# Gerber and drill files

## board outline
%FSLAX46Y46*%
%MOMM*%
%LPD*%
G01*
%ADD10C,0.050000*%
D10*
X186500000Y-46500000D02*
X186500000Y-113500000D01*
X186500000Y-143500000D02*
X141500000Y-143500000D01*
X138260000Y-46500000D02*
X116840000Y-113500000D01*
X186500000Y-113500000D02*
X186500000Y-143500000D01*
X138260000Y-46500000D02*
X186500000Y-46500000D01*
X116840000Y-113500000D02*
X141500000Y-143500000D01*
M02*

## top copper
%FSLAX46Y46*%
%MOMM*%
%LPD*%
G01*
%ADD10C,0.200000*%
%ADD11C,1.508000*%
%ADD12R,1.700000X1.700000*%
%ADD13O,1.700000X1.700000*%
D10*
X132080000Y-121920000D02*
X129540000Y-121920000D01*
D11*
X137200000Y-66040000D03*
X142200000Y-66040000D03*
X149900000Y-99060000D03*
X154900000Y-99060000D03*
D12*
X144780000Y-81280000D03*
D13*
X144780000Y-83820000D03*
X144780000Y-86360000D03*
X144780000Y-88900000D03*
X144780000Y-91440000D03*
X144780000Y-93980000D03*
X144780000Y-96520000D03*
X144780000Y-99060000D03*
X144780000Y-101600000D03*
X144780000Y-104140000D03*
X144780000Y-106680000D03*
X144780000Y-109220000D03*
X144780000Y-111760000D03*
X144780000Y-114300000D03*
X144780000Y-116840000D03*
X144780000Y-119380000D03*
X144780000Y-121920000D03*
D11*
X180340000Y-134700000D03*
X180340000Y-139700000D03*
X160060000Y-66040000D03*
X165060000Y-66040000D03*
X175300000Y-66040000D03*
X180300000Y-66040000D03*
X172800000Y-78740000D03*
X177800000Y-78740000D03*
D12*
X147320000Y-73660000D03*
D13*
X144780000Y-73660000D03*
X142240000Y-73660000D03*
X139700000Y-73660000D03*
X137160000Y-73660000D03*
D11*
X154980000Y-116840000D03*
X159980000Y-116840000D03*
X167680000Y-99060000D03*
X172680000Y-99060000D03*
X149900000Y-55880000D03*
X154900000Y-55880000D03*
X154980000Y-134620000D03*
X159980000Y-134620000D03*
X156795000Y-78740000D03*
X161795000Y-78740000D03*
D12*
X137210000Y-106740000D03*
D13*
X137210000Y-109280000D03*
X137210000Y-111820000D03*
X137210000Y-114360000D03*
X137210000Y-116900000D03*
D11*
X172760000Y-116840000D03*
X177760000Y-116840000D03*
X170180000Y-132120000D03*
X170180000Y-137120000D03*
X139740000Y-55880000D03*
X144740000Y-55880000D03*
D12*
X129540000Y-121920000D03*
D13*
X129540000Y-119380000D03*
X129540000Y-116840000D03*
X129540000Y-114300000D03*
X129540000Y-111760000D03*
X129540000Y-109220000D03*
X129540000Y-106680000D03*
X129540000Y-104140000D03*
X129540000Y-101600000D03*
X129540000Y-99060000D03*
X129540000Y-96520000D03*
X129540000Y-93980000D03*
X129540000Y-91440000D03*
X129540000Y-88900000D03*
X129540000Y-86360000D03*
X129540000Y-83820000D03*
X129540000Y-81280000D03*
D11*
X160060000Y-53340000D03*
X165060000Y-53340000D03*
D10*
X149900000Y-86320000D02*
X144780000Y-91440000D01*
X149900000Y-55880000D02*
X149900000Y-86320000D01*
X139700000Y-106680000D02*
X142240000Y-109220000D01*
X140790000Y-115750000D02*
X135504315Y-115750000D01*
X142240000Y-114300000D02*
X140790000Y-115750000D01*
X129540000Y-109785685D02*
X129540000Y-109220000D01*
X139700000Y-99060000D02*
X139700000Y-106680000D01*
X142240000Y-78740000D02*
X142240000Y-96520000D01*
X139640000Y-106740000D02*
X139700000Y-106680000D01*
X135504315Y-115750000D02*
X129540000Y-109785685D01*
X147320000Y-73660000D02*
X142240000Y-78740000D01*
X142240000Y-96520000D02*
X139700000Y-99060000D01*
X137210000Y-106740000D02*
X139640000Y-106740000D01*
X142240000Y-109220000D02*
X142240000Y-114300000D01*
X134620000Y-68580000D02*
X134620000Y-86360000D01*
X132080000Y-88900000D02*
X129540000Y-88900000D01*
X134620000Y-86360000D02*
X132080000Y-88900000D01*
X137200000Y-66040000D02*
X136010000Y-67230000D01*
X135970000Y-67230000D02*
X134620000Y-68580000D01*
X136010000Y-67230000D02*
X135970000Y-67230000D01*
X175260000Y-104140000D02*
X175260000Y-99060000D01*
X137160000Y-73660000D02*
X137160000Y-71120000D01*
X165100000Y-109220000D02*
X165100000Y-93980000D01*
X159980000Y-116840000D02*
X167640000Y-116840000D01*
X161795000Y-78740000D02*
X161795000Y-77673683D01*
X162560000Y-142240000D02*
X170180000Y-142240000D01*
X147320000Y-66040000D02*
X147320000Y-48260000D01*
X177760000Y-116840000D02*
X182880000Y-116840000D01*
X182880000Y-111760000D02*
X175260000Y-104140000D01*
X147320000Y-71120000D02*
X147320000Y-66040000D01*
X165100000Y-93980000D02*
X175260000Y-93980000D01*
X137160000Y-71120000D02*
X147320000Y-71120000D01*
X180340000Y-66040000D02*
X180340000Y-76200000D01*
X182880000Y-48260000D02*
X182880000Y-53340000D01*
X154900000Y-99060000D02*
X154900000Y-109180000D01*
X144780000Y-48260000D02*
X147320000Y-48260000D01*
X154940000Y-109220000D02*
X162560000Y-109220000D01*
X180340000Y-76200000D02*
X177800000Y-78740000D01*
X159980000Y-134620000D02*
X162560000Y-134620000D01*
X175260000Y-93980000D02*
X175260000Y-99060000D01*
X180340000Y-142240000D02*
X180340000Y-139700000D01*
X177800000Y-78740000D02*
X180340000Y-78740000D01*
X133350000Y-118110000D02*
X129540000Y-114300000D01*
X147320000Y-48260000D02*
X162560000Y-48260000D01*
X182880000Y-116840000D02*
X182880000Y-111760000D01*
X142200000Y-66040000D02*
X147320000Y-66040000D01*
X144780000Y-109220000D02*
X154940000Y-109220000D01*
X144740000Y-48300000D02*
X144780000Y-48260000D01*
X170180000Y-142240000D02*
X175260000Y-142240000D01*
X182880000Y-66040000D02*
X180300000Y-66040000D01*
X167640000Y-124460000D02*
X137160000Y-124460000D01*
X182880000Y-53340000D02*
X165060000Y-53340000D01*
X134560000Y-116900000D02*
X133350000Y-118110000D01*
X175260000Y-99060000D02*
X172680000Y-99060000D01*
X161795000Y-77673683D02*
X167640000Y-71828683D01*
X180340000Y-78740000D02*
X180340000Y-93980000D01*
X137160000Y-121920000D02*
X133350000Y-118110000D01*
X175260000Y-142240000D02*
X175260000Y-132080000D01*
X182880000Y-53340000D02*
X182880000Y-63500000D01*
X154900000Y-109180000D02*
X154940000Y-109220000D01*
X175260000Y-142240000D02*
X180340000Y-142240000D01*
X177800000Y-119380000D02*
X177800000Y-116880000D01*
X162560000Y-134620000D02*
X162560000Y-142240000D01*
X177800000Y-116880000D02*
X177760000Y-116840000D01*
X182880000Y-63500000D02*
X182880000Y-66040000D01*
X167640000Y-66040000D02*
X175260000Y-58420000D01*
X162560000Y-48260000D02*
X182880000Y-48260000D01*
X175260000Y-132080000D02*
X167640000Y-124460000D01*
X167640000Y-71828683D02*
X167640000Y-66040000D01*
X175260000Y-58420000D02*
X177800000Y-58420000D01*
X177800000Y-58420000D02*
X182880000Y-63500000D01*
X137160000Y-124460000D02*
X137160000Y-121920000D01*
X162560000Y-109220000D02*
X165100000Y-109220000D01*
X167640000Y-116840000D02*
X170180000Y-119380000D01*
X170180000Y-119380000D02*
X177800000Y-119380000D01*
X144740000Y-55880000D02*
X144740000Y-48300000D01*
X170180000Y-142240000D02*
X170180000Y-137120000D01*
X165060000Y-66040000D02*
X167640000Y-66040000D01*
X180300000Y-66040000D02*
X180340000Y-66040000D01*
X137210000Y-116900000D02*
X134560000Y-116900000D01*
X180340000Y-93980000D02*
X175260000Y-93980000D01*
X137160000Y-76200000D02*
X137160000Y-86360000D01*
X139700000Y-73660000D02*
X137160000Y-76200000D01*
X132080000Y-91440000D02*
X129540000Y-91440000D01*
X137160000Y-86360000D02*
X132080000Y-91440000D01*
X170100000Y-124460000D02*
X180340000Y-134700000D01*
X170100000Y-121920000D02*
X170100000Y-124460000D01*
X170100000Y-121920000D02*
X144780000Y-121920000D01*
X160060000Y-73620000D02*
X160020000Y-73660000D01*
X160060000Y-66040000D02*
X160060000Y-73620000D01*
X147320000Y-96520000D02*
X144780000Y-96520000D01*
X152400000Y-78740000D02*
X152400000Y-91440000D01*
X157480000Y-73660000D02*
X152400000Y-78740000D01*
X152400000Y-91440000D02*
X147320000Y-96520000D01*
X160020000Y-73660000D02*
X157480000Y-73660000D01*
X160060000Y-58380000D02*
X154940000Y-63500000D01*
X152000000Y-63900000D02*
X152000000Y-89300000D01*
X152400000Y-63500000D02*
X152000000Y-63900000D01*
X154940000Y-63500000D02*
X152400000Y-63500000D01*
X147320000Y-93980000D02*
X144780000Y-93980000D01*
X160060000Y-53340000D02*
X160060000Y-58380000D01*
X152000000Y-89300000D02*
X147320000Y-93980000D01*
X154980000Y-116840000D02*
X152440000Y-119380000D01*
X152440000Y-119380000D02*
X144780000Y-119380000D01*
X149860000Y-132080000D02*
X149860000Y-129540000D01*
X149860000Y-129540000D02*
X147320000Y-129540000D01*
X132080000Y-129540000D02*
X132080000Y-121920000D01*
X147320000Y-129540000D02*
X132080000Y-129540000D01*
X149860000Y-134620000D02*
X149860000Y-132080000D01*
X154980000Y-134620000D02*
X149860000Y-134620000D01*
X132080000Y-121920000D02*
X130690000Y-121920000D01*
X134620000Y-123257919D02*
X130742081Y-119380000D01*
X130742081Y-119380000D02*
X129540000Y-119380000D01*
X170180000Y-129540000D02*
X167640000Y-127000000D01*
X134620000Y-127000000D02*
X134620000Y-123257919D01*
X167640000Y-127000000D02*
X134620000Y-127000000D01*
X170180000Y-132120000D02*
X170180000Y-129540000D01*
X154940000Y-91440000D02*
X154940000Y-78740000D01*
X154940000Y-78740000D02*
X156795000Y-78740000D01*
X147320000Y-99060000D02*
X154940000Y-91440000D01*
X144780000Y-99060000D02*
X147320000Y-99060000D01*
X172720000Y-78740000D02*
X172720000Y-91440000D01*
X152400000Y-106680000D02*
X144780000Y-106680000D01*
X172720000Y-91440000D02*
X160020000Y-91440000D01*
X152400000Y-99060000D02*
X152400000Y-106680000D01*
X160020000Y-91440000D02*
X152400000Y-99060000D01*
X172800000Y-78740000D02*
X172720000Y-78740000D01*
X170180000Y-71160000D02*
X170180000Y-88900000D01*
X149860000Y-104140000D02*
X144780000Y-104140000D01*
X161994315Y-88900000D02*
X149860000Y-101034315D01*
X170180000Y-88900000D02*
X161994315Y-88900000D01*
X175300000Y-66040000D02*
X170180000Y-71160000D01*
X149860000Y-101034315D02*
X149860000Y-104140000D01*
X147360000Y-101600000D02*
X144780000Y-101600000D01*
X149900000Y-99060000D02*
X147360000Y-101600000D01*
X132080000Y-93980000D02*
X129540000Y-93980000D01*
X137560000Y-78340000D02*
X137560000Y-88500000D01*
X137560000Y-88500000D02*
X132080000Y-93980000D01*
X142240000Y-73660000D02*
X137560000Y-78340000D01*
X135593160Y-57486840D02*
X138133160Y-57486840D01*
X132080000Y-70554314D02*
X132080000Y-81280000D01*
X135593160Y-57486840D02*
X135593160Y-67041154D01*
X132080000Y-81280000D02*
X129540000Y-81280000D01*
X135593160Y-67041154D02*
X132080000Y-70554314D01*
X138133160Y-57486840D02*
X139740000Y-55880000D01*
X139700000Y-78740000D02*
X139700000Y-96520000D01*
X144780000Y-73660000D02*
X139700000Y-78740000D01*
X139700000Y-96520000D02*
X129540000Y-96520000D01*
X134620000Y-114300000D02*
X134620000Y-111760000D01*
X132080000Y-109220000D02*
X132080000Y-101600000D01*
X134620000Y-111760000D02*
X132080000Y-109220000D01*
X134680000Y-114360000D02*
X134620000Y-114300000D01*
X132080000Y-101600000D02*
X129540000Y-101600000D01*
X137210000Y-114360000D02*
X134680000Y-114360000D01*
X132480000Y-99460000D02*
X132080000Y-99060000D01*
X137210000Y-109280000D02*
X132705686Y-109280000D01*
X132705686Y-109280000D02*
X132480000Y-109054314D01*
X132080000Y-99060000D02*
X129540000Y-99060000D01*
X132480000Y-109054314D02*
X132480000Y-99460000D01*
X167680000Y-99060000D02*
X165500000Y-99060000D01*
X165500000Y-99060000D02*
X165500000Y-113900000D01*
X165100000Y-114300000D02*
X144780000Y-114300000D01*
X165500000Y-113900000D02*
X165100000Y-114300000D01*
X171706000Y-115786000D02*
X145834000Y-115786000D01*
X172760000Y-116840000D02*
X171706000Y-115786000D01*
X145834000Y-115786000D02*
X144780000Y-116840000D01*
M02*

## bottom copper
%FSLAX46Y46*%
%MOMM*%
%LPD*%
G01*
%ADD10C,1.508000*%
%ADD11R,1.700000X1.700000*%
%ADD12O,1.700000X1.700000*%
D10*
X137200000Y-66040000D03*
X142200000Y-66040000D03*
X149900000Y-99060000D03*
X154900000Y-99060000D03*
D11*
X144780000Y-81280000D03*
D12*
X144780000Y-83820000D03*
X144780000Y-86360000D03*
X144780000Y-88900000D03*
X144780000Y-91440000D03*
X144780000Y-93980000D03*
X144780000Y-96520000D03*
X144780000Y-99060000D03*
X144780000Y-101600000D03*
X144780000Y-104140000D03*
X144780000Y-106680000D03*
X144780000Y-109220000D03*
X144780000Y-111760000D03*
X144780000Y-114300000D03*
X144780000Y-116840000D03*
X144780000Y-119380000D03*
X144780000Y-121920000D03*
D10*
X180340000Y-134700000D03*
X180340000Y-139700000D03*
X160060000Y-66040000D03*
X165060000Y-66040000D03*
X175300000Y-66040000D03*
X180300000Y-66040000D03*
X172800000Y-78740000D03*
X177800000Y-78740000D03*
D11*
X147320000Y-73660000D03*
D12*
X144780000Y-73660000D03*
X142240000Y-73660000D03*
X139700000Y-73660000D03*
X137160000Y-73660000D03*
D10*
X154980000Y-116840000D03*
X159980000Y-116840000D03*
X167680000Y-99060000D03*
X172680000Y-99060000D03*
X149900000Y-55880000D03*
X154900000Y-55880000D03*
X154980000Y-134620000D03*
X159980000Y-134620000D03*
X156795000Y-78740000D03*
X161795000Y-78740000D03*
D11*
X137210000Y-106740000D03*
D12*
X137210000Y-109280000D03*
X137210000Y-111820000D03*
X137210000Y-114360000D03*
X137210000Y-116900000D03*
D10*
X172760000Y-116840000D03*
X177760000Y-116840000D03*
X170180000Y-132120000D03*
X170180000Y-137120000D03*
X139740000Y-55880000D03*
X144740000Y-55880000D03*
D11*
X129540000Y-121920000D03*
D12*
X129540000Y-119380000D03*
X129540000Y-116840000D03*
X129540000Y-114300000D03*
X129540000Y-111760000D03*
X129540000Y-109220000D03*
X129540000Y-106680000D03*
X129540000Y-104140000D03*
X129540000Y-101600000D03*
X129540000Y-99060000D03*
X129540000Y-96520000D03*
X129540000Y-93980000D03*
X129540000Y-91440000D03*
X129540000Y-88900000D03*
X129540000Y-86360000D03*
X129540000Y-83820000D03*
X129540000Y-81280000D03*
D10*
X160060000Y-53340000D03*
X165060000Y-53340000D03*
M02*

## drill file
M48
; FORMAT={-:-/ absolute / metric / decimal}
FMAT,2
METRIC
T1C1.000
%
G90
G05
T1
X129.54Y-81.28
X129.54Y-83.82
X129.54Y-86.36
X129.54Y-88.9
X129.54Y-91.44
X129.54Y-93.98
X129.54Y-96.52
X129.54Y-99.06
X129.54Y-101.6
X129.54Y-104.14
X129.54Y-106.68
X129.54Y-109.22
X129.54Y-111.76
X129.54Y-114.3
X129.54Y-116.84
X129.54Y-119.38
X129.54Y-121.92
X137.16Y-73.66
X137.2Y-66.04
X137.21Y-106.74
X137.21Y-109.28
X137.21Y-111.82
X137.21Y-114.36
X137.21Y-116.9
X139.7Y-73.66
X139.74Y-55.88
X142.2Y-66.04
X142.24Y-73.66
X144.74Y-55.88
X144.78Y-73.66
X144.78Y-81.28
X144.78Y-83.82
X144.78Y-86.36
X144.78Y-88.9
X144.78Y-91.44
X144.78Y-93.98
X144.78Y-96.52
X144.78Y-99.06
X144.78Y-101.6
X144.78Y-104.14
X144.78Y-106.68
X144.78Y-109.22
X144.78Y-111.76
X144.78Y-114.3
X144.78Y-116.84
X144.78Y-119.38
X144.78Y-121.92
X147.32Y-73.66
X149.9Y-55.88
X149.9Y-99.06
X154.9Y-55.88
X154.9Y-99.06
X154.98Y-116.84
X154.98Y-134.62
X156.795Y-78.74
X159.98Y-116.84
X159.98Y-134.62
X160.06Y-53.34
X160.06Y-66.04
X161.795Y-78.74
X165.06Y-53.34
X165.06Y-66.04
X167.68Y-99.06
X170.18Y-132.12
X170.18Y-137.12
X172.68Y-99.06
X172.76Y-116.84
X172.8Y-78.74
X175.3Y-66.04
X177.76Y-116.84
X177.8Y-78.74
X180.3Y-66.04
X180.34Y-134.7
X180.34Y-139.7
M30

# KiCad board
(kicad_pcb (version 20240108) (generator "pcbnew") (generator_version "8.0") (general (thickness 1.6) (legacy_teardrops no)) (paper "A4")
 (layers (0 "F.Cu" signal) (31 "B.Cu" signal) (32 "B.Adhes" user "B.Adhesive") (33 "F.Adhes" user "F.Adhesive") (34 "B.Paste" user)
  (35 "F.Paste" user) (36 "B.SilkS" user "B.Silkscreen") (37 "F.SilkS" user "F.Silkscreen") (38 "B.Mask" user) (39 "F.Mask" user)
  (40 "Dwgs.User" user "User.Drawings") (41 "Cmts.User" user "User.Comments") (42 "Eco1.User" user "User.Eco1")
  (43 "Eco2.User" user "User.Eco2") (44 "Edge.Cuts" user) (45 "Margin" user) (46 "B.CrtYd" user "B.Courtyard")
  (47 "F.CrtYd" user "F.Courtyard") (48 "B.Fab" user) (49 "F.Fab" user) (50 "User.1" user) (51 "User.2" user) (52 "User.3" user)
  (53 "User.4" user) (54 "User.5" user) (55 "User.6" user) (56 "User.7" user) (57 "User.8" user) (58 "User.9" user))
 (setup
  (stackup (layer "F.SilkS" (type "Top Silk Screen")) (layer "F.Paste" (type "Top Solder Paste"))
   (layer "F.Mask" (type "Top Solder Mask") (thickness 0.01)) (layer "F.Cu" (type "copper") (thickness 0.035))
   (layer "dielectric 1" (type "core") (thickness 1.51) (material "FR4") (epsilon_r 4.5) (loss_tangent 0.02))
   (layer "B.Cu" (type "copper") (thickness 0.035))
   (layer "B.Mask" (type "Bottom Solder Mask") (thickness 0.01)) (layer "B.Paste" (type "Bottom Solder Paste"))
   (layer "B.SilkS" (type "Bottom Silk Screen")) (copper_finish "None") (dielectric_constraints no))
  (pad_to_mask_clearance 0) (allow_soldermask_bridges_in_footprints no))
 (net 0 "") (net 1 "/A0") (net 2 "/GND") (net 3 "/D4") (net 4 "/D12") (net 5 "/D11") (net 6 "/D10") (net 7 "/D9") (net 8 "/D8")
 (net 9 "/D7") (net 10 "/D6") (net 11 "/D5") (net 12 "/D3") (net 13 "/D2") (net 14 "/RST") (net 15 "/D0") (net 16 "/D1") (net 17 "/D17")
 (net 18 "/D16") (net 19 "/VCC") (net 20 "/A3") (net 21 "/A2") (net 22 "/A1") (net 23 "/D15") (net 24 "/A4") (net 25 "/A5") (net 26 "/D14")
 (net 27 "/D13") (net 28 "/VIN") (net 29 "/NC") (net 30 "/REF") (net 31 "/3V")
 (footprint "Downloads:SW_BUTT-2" (layer "F.Cu") (at 139.7 66.04)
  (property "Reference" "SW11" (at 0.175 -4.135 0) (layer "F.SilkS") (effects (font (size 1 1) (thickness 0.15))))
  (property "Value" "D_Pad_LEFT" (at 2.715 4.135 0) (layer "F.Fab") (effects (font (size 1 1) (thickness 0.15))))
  (pad "1" thru_hole circle (at -2.5 0) (size 1.508 1.508) (drill 1) (layers "*.Cu" "*.Mask") (remove_unused_layers no) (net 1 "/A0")
   (solder_mask_margin 0.102))
  (pad "2" thru_hole circle (at 2.5 0) (size 1.508 1.508) (drill 1) (layers "*.Cu" "*.Mask") (remove_unused_layers no) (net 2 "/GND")
   (solder_mask_margin 0.102)))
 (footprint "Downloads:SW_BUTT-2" (layer "F.Cu") (at 152.4 99.06)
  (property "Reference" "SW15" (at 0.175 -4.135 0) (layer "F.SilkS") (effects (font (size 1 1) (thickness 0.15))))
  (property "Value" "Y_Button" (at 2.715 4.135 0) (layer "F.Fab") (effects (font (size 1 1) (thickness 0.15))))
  (pad "1" thru_hole circle (at -2.5 0) (size 1.508 1.508) (drill 1) (layers "*.Cu" "*.Mask") (remove_unused_layers no) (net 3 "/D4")
   (solder_mask_margin 0.102))
  (pad "2" thru_hole circle (at 2.5 0) (size 1.508 1.508) (drill 1) (layers "*.Cu" "*.Mask") (remove_unused_layers no) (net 2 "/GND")
   (solder_mask_margin 0.102)))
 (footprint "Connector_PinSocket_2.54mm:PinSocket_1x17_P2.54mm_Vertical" (layer "F.Cu") (at 144.78 81.28)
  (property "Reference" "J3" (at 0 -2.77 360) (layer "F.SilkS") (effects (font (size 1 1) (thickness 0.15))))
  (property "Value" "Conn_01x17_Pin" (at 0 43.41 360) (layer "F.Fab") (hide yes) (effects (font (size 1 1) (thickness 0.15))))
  (pad "1" thru_hole rect (at 0 0) (size 1.7 1.7) (drill 1) (layers "*.Cu" "*.Mask") (remove_unused_layers no) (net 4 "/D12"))
  (pad "2" thru_hole oval (at 0 2.54) (size 1.7 1.7) (drill 1) (layers "*.Cu" "*.Mask") (remove_unused_layers no) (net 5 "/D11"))
  (pad "3" thru_hole oval (at 0 5.08) (size 1.7 1.7) (drill 1) (layers "*.Cu" "*.Mask") (remove_unused_layers no) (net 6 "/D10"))
  (pad "4" thru_hole oval (at 0 7.62) (size 1.7 1.7) (drill 1) (layers "*.Cu" "*.Mask") (remove_unused_layers no) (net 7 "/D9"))
  (pad "5" thru_hole oval (at 0 10.16) (size 1.7 1.7) (drill 1) (layers "*.Cu" "*.Mask") (remove_unused_layers no) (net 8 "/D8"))
  (pad "6" thru_hole oval (at 0 12.7) (size 1.7 1.7) (drill 1) (layers "*.Cu" "*.Mask") (remove_unused_layers no) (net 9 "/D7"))
  (pad "7" thru_hole oval (at 0 15.24) (size 1.7 1.7) (drill 1) (layers "*.Cu" "*.Mask") (remove_unused_layers no) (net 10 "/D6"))
  (pad "8" thru_hole oval (at 0 17.78) (size 1.7 1.7) (drill 1) (layers "*.Cu" "*.Mask") (remove_unused_layers no) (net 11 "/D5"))
  (pad "9" thru_hole oval (at 0 20.32) (size 1.7 1.7) (drill 1) (layers "*.Cu" "*.Mask") (remove_unused_layers no) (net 3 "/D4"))
  (pad "10" thru_hole oval (at 0 22.86) (size 1.7 1.7) (drill 1) (layers "*.Cu" "*.Mask") (remove_unused_layers no) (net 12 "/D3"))
  (pad "11" thru_hole oval (at 0 25.4) (size 1.7 1.7) (drill 1) (layers "*.Cu" "*.Mask") (remove_unused_layers no) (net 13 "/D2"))
  (pad "12" thru_hole oval (at 0 27.94) (size 1.7 1.7) (drill 1) (layers "*.Cu" "*.Mask") (remove_unused_layers no) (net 2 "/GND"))
  (pad "13" thru_hole oval (at 0 30.48) (size 1.7 1.7) (drill 1) (layers "*.Cu" "*.Mask") (remove_unused_layers no) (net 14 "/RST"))
  (pad "14" thru_hole oval (at 0 33.02) (size 1.7 1.7) (drill 1) (layers "*.Cu" "*.Mask") (remove_unused_layers no) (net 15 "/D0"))
  (pad "15" thru_hole oval (at 0 35.56) (size 1.7 1.7) (drill 1) (layers "*.Cu" "*.Mask") (remove_unused_layers no) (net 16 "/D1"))
  (pad "16" thru_hole oval (at 0 38.1) (size 1.7 1.7) (drill 1) (layers "*.Cu" "*.Mask") (remove_unused_layers no) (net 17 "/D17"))
  (pad "17" thru_hole oval (at 0 40.64) (size 1.7 1.7) (drill 1) (layers "*.Cu" "*.Mask") (remove_unused_layers no) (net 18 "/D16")))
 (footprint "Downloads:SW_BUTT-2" (layer "F.Cu") (at 180.34 137.2 -90)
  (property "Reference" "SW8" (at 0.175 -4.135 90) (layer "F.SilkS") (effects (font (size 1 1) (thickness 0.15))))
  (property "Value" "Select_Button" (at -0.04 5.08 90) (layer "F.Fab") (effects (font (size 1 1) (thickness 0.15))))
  (pad "1" thru_hole circle (at -2.5 0 270) (size 1.508 1.508) (drill 1) (layers "*.Cu" "*.Mask") (remove_unused_layers no) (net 18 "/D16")
   (solder_mask_margin 0.102))
  (pad "2" thru_hole circle (at 2.5 0 270) (size 1.508 1.508) (drill 1) (layers "*.Cu" "*.Mask") (remove_unused_layers no) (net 2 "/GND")
   (solder_mask_margin 0.102)))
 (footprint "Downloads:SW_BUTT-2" (layer "F.Cu") (at 162.56 66.04)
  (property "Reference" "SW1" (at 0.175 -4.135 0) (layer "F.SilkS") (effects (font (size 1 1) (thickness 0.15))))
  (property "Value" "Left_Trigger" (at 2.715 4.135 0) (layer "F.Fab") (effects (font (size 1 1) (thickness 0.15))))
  (pad "1" thru_hole circle (at -2.5 0) (size 1.508 1.508) (drill 1) (layers "*.Cu" "*.Mask") (remove_unused_layers no) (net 10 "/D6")
   (solder_mask_margin 0.102))
  (pad "2" thru_hole circle (at 2.5 0) (size 1.508 1.508) (drill 1) (layers "*.Cu" "*.Mask") (remove_unused_layers no) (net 2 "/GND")
   (solder_mask_margin 0.102)))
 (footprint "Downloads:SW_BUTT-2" (layer "F.Cu") (at 177.8 66.04)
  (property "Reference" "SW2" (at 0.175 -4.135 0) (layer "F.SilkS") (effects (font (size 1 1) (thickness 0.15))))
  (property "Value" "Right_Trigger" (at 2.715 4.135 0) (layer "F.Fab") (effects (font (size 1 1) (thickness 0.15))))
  (pad "1" thru_hole circle (at -2.5 0) (size 1.508 1.508) (drill 1) (layers "*.Cu" "*.Mask") (remove_unused_layers no) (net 12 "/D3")
   (solder_mask_margin 0.102))
  (pad "2" thru_hole circle (at 2.5 0) (size 1.508 1.508) (drill 1) (layers "*.Cu" "*.Mask") (remove_unused_layers no) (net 2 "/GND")
   (solder_mask_margin 0.102)))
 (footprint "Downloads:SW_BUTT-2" (layer "F.Cu") (at 175.3 78.74)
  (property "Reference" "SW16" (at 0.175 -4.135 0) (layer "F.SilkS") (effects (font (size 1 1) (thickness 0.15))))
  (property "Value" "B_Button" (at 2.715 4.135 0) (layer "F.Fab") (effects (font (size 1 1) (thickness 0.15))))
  (pad "1" thru_hole circle (at -2.5 0) (size 1.508 1.508) (drill 1) (layers "*.Cu" "*.Mask") (remove_unused_layers no) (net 13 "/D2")
   (solder_mask_margin 0.102))
  (pad "2" thru_hole circle (at 2.5 0) (size 1.508 1.508) (drill 1) (layers "*.Cu" "*.Mask") (remove_unused_layers no) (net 2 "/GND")
   (solder_mask_margin 0.102)))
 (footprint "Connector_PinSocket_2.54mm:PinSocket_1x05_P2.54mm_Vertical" (layer "F.Cu") (at 147.32 73.66 -90)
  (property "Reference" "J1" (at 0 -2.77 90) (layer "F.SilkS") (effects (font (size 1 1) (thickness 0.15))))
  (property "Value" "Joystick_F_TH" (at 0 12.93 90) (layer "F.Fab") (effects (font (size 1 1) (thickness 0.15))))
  (pad "1" thru_hole rect (at 0 0 270) (size 1.7 1.7) (drill 1) (layers "*.Cu" "*.Mask") (remove_unused_layers no) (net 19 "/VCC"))
  (pad "2" thru_hole oval (at 0 2.54 270) (size 1.7 1.7) (drill 1) (layers "*.Cu" "*.Mask") (remove_unused_layers no) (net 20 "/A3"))
  (pad "3" thru_hole oval (at 0 5.08 270) (size 1.7 1.7) (drill 1) (layers "*.Cu" "*.Mask") (remove_unused_layers no) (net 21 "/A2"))
  (pad "4" thru_hole oval (at 0 7.62 270) (size 1.7 1.7) (drill 1) (layers "*.Cu" "*.Mask") (remove_unused_layers no) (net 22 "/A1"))
  (pad "5" thru_hole oval (at 0 10.16 270) (size 1.7 1.7) (drill 1) (layers "*.Cu" "*.Mask") (remove_unused_layers no) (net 2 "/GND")))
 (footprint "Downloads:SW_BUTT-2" (layer "F.Cu") (at 157.48 116.84)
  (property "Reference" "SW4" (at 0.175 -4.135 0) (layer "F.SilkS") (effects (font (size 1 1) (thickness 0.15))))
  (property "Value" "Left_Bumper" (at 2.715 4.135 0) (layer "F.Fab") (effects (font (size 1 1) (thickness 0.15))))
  (pad "1" thru_hole circle (at -2.5 0) (size 1.508 1.508) (drill 1) (layers "*.Cu" "*.Mask") (remove_unused_layers no) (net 17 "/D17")
   (solder_mask_margin 0.102))
  (pad "2" thru_hole circle (at 2.5 0) (size 1.508 1.508) (drill 1) (layers "*.Cu" "*.Mask") (remove_unused_layers no) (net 2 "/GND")
   (solder_mask_margin 0.102)))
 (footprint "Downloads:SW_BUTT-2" (layer "F.Cu") (at 170.18 99.06)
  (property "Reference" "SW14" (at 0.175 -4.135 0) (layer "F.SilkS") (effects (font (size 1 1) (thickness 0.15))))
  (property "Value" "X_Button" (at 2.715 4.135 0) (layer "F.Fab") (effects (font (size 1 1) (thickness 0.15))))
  (pad "1" thru_hole circle (at -2.5 0) (size 1.508 1.508) (drill 1) (layers "*.Cu" "*.Mask") (remove_unused_layers no) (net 15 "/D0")
   (solder_mask_margin 0.102))
  (pad "2" thru_hole circle (at 2.5 0) (size 1.508 1.508) (drill 1) (layers "*.Cu" "*.Mask") (remove_unused_layers no) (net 2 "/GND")
   (solder_mask_margin 0.102)))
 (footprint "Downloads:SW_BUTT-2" (layer "F.Cu") (at 152.4 55.88)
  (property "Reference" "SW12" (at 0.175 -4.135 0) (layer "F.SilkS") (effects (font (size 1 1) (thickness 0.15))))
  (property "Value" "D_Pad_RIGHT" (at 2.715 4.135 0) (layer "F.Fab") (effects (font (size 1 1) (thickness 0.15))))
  (pad "1" thru_hole circle (at -2.5 0) (size 1.508 1.508) (drill 1) (layers "*.Cu" "*.Mask") (remove_unused_layers no) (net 8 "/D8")
   (solder_mask_margin 0.102))
  (pad "2" thru_hole circle (at 2.5 0) (size 1.508 1.508) (drill 1) (layers "*.Cu" "*.Mask") (remove_unused_layers no) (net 2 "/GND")
   (solder_mask_margin 0.102)))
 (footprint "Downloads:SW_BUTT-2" (layer "F.Cu") (at 157.48 134.62)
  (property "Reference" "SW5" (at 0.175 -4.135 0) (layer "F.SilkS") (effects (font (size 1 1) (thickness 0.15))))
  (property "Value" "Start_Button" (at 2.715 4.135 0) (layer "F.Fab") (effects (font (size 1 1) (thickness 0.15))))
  (pad "1" thru_hole circle (at -2.5 0) (size 1.508 1.508) (drill 1) (layers "*.Cu" "*.Mask") (remove_unused_layers no) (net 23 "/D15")
   (solder_mask_margin 0.102))
  (pad "2" thru_hole circle (at 2.5 0) (size 1.508 1.508) (drill 1) (layers "*.Cu" "*.Mask") (remove_unused_layers no) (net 2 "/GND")
   (solder_mask_margin 0.102)))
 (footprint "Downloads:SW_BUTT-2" (layer "F.Cu") (at 159.295 78.74)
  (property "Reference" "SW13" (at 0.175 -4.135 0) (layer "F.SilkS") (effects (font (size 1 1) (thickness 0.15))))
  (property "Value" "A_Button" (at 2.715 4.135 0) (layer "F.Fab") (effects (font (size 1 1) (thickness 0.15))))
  (pad "1" thru_hole circle (at -2.5 0) (size 1.508 1.508) (drill 1) (layers "*.Cu" "*.Mask") (remove_unused_layers no) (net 11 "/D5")
   (solder_mask_margin 0.102))
  (pad "2" thru_hole circle (at 2.5 0) (size 1.508 1.508) (drill 1) (layers "*.Cu" "*.Mask") (remove_unused_layers no) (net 2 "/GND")
   (solder_mask_margin 0.102)))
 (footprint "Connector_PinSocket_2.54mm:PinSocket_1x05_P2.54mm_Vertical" (layer "F.Cu") (at 137.21 106.74)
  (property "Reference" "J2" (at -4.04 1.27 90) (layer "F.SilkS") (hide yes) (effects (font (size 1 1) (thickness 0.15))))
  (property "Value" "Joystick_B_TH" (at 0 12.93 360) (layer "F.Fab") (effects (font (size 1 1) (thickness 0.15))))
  (pad "1" thru_hole rect (at 0 0) (size 1.7 1.7) (drill 1) (layers "*.Cu" "*.Mask") (remove_unused_layers no) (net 19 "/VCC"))
  (pad "2" thru_hole oval (at 0 2.54) (size 1.7 1.7) (drill 1) (layers "*.Cu" "*.Mask") (remove_unused_layers no) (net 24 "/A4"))
  (pad "3" thru_hole oval (at 0 5.08) (size 1.7 1.7) (drill 1) (layers "*.Cu" "*.Mask") (remove_unused_layers no) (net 9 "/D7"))
  (pad "4" thru_hole oval (at 0 7.62) (size 1.7 1.7) (drill 1) (layers "*.Cu" "*.Mask") (remove_unused_layers no) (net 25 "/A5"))
  (pad "5" thru_hole oval (at 0 10.16) (size 1.7 1.7) (drill 1) (layers "*.Cu" "*.Mask") (remove_unused_layers no) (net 2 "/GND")))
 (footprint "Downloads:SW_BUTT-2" (layer "F.Cu") (at 175.26 116.84)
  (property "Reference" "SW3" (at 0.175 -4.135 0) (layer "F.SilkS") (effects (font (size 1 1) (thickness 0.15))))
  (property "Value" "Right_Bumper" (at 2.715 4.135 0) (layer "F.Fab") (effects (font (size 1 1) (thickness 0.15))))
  (pad "1" thru_hole circle (at -2.5 0) (size 1.508 1.508) (drill 1) (layers "*.Cu" "*.Mask") (remove_unused_layers no) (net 16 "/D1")
   (solder_mask_margin 0.102))
  (pad "2" thru_hole circle (at 2.5 0) (size 1.508 1.508) (drill 1) (layers "*.Cu" "*.Mask") (remove_unused_layers no) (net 2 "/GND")
   (solder_mask_margin 0.102)))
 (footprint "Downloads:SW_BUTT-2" (layer "F.Cu") (at 170.18 134.62 -90)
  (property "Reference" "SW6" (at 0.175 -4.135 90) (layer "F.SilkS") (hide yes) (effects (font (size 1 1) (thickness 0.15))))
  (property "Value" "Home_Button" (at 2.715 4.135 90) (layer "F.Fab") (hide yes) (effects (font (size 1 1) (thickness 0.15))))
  (pad "1" thru_hole circle (at -2.5 0 270) (size 1.508 1.508) (drill 1) (layers "*.Cu" "*.Mask") (remove_unused_layers no) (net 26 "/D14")
   (solder_mask_margin 0.102))
  (pad "2" thru_hole circle (at 2.5 0 270) (size 1.508 1.508) (drill 1) (layers "*.Cu" "*.Mask") (remove_unused_layers no) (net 2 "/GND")
   (solder_mask_margin 0.102)))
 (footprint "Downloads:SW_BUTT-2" (layer "F.Cu") (at 142.24 55.88)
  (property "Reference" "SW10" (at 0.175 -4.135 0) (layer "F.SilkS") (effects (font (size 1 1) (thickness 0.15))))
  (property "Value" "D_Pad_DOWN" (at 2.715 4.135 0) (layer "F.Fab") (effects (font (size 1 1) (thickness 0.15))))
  (pad "1" thru_hole circle (at -2.5 0) (size 1.508 1.508) (drill 1) (layers "*.Cu" "*.Mask") (remove_unused_layers no) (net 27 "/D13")
   (solder_mask_margin 0.102))
  (pad "2" thru_hole circle (at 2.5 0) (size 1.508 1.508) (drill 1) (layers "*.Cu" "*.Mask") (remove_unused_layers no) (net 2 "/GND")
   (solder_mask_margin 0.102)))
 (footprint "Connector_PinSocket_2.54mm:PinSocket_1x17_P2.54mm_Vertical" (layer "F.Cu") (at 129.54 121.92 180)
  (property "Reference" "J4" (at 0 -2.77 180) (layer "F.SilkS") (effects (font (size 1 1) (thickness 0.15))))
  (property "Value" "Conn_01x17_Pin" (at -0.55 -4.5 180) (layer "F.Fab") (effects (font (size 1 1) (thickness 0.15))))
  (pad "1" thru_hole rect (at 0 0 180) (size 1.7 1.7) (drill 1) (layers "*.Cu" "*.Mask") (remove_unused_layers no) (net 23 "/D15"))
  (pad "2" thru_hole oval (at 0 2.54 180) (size 1.7 1.7) (drill 1) (layers "*.Cu" "*.Mask") (remove_unused_layers no) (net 26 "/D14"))
  (pad "3" thru_hole oval (at 0 5.08 180) (size 1.7 1.7) (drill 1) (layers "*.Cu" "*.Mask") (remove_unused_layers no) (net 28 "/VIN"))
  (pad "4" thru_hole oval (at 0 7.62 180) (size 1.7 1.7) (drill 1) (layers "*.Cu" "*.Mask") (remove_unused_layers no) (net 2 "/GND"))
  (pad "5" thru_hole oval (at 0 10.16 180) (size 1.7 1.7) (drill 1) (layers "*.Cu" "*.Mask") (remove_unused_layers no) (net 14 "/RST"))
  (pad "6" thru_hole oval (at 0 12.7 180) (size 1.7 1.7) (drill 1) (layers "*.Cu" "*.Mask") (remove_unused_layers no) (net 19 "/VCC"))
  (pad "7" thru_hole oval (at 0 15.24 180) (size 1.7 1.7) (drill 1) (layers "*.Cu" "*.Mask") (remove_unused_layers no) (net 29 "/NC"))
  (pad "8" thru_hole oval (at 0 17.78 180) (size 1.7 1.7) (drill 1) (layers "*.Cu" "*.Mask") (remove_unused_layers no) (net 29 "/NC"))
  (pad "9" thru_hole oval (at 0 20.32 180) (size 1.7 1.7) (drill 1) (layers "*.Cu" "*.Mask") (remove_unused_layers no) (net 25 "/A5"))
  (pad "10" thru_hole oval (at 0 22.86 180) (size 1.7 1.7) (drill 1) (layers "*.Cu" "*.Mask") (remove_unused_layers no) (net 24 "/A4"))
  (pad "11" thru_hole oval (at 0 25.4 180) (size 1.7 1.7) (drill 1) (layers "*.Cu" "*.Mask") (remove_unused_layers no) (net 20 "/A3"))
  (pad "12" thru_hole oval (at 0 27.94 180) (size 1.7 1.7) (drill 1) (layers "*.Cu" "*.Mask") (remove_unused_layers no) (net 21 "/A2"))
  (pad "13" thru_hole oval (at 0 30.48 180) (size 1.7 1.7) (drill 1) (layers "*.Cu" "*.Mask") (remove_unused_layers no) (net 22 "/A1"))
  (pad "14" thru_hole oval (at 0 33.02 180) (size 1.7 1.7) (drill 1) (layers "*.Cu" "*.Mask") (remove_unused_layers no) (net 1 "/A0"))
  (pad "15" thru_hole oval (at 0 35.56 180) (size 1.7 1.7) (drill 1) (layers "*.Cu" "*.Mask") (remove_unused_layers no) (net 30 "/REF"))
  (pad "16" thru_hole oval (at 0 38.1 180) (size 1.7 1.7) (drill 1) (layers "*.Cu" "*.Mask") (remove_unused_layers no) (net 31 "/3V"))
  (pad "17" thru_hole oval (at 0 40.64 180) (size 1.7 1.7) (drill 1) (layers "*.Cu" "*.Mask") (remove_unused_layers no) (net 27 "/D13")))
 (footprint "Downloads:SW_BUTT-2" (layer "F.Cu") (at 162.56 53.34)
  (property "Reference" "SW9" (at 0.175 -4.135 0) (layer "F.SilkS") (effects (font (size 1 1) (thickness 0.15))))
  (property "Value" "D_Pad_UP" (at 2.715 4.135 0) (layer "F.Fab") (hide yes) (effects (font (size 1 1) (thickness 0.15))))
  (pad "1" thru_hole circle (at -2.5 0) (size 1.508 1.508) (drill 1) (layers "*.Cu" "*.Mask") (remove_unused_layers no) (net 9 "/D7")
   (solder_mask_margin 0.102))
  (pad "2" thru_hole circle (at 2.5 0) (size 1.508 1.508) (drill 1) (layers "*.Cu" "*.Mask") (remove_unused_layers no) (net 2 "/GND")
   (solder_mask_margin 0.102)))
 (gr_line (start 132.08 121.92) (end 129.54 121.92) (stroke (width 0.2) (type default)) (layer "F.Cu") (net 23))
 (gr_line (start 186.5 46.5) (end 186.5 113.5) (stroke (width 0.05) (type default)) (layer "Edge.Cuts"))
 (gr_line (start 186.5 143.5) (end 141.5 143.5) (stroke (width 0.05) (type default)) (layer "Edge.Cuts"))
 (gr_line (start 138.26 46.5) (end 116.84 113.5) (stroke (width 0.05) (type default)) (layer "Edge.Cuts"))
 (gr_line (start 186.5 113.5) (end 186.5 143.5) (stroke (width 0.05) (type default)) (layer "Edge.Cuts"))
 (gr_line (start 138.26 46.5) (end 186.5 46.5) (stroke (width 0.05) (type default)) (layer "Edge.Cuts"))
 (gr_line (start 116.84 113.5) (end 141.5 143.5) (stroke (width 0.05) (type default)) (layer "Edge.Cuts"))
 (segment (start 149.9 86.32) (end 144.78 91.44) (width 0.2) (layer "F.Cu") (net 8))
 (segment (start 149.9 55.88) (end 149.9 86.32) (width 0.2) (layer "F.Cu") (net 8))
 (segment (start 139.7 106.68) (end 142.24 109.22) (width 0.2) (layer "F.Cu") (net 19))
 (segment (start 140.79 115.75) (end 135.504315 115.75) (width 0.2) (layer "F.Cu") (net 19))
 (segment (start 142.24 114.3) (end 140.79 115.75) (width 0.2) (layer "F.Cu") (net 19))
 (segment (start 129.54 109.785685) (end 129.54 109.22) (width 0.2) (layer "F.Cu") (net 19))
 (segment (start 139.7 99.06) (end 139.7 106.68) (width 0.2) (layer "F.Cu") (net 19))
 (segment (start 142.24 78.74) (end 142.24 96.52) (width 0.2) (layer "F.Cu") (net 19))
 (segment (start 139.64 106.74) (end 139.7 106.68) (width 0.2) (layer "F.Cu") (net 19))
 (segment (start 135.504315 115.75) (end 129.54 109.785685) (width 0.2) (layer "F.Cu") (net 19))
 (segment (start 147.32 73.66) (end 142.24 78.74) (width 0.2) (layer "F.Cu") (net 19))
 (segment (start 142.24 96.52) (end 139.7 99.06) (width 0.2) (layer "F.Cu") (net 19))
 (segment (start 137.21 106.74) (end 139.64 106.74) (width 0.2) (layer "F.Cu") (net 19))
 (segment (start 142.24 109.22) (end 142.24 114.3) (width 0.2) (layer "F.Cu") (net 19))
 (segment (start 134.62 68.58) (end 134.62 86.36) (width 0.2) (layer "F.Cu") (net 1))
 (segment (start 132.08 88.9) (end 129.54 88.9) (width 0.2) (layer "F.Cu") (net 1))
 (segment (start 134.62 86.36) (end 132.08 88.9) (width 0.2) (layer "F.Cu") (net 1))
 (segment (start 137.2 66.04) (end 136.01 67.23) (width 0.2) (layer "F.Cu") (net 1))
 (segment (start 135.97 67.23) (end 134.62 68.58) (width 0.2) (layer "F.Cu") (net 1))
 (segment (start 136.01 67.23) (end 135.97 67.23) (width 0.2) (layer "F.Cu") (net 1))
 (segment (start 175.26 104.14) (end 175.26 99.06) (width 0.2) (layer "F.Cu") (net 2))
 (segment (start 137.16 73.66) (end 137.16 71.12) (width 0.2) (layer "F.Cu") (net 2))
 (segment (start 165.1 109.22) (end 165.1 93.98) (width 0.2) (layer "F.Cu") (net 2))
 (segment (start 159.98 116.84) (end 167.64 116.84) (width 0.2) (layer "F.Cu") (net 2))
 (segment (start 161.795 78.74) (end 161.795 77.673683) (width 0.2) (layer "F.Cu") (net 2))
 (segment (start 162.56 142.24) (end 170.18 142.24) (width 0.2) (layer "F.Cu") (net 2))
 (segment (start 147.32 66.04) (end 147.32 48.26) (width 0.2) (layer "F.Cu") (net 2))
 (segment (start 177.76 116.84) (end 182.88 116.84) (width 0.2) (layer "F.Cu") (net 2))
 (segment (start 182.88 111.76) (end 175.26 104.14) (width 0.2) (layer "F.Cu") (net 2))
 (segment (start 147.32 71.12) (end 147.32 66.04) (width 0.2) (layer "F.Cu") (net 2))
 (segment (start 165.1 93.98) (end 175.26 93.98) (width 0.2) (layer "F.Cu") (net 2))
 (segment (start 137.16 71.12) (end 147.32 71.12) (width 0.2) (layer "F.Cu") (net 2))
 (segment (start 180.34 66.04) (end 180.34 76.2) (width 0.2) (layer "F.Cu") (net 2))
 (segment (start 182.88 48.26) (end 182.88 53.34) (width 0.2) (layer "F.Cu") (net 2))
 (segment (start 154.9 99.06) (end 154.9 109.18) (width 0.2) (layer "F.Cu") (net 2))
 (segment (start 144.78 48.26) (end 147.32 48.26) (width 0.2) (layer "F.Cu") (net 2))
 (segment (start 154.94 109.22) (end 162.56 109.22) (width 0.2) (layer "F.Cu") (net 2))
 (segment (start 180.34 76.2) (end 177.8 78.74) (width 0.2) (layer "F.Cu") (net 2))
 (segment (start 159.98 134.62) (end 162.56 134.62) (width 0.2) (layer "F.Cu") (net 2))
 (segment (start 175.26 93.98) (end 175.26 99.06) (width 0.2) (layer "F.Cu") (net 2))
 (segment (start 180.34 142.24) (end 180.34 139.7) (width 0.2) (layer "F.Cu") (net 2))
 (segment (start 177.8 78.74) (end 180.34 78.74) (width 0.2) (layer "F.Cu") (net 2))
 (segment (start 133.35 118.11) (end 129.54 114.3) (width 0.2) (layer "F.Cu") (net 2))
 (segment (start 147.32 48.26) (end 162.56 48.26) (width 0.2) (layer "F.Cu") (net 2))
 (segment (start 182.88 116.84) (end 182.88 111.76) (width 0.2) (layer "F.Cu") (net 2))
 (segment (start 142.2 66.04) (end 147.32 66.04) (width 0.2) (layer "F.Cu") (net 2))
 (segment (start 144.78 109.22) (end 154.94 109.22) (width 0.2) (layer "F.Cu") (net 2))
 (segment (start 144.74 48.3) (end 144.78 48.26) (width 0.2) (layer "F.Cu") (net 2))
 (segment (start 170.18 142.24) (end 175.26 142.24) (width 0.2) (layer "F.Cu") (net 2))
 (segment (start 182.88 66.04) (end 180.3 66.04) (width 0.2) (layer "F.Cu") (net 2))
 (segment (start 167.64 124.46) (end 137.16 124.46) (width 0.2) (layer "F.Cu") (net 2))
 (segment (start 182.88 53.34) (end 165.06 53.34) (width 0.2) (layer "F.Cu") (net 2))
 (segment (start 134.56 116.9) (end 133.35 118.11) (width 0.2) (layer "F.Cu") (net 2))
 (segment (start 175.26 99.06) (end 172.68 99.06) (width 0.2) (layer "F.Cu") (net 2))
 (segment (start 161.795 77.673683) (end 167.64 71.828683) (width 0.2) (layer "F.Cu") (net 2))
 (segment (start 180.34 78.74) (end 180.34 93.98) (width 0.2) (layer "F.Cu") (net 2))
 (segment (start 137.16 121.92) (end 133.35 118.11) (width 0.2) (layer "F.Cu") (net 2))
 (segment (start 175.26 142.24) (end 175.26 132.08) (width 0.2) (layer "F.Cu") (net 2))
 (segment (start 182.88 53.34) (end 182.88 63.5) (width 0.2) (layer "F.Cu") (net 2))
 (segment (start 154.9 109.18) (end 154.94 109.22) (width 0.2) (layer "F.Cu") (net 2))
 (segment (start 175.26 142.24) (end 180.34 142.24) (width 0.2) (layer "F.Cu") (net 2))
 (segment (start 177.8 119.38) (end 177.8 116.88) (width 0.2) (layer "F.Cu") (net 2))
 (segment (start 162.56 134.62) (end 162.56 142.24) (width 0.2) (layer "F.Cu") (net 2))
 (segment (start 177.8 116.88) (end 177.76 116.84) (width 0.2) (layer "F.Cu") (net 2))
 (segment (start 182.88 63.5) (end 182.88 66.04) (width 0.2) (layer "F.Cu") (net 2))
 (segment (start 167.64 66.04) (end 175.26 58.42) (width 0.2) (layer "F.Cu") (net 2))
 (segment (start 162.56 48.26) (end 182.88 48.26) (width 0.2) (layer "F.Cu") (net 2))
 (segment (start 175.26 132.08) (end 167.64 124.46) (width 0.2) (layer "F.Cu") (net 2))
 (segment (start 167.64 71.828683) (end 167.64 66.04) (width 0.2) (layer "F.Cu") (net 2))
 (segment (start 175.26 58.42) (end 177.8 58.42) (width 0.2) (layer "F.Cu") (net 2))
 (segment (start 177.8 58.42) (end 182.88 63.5) (width 0.2) (layer "F.Cu") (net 2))
 (segment (start 137.16 124.46) (end 137.16 121.92) (width 0.2) (layer "F.Cu") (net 2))
 (segment (start 162.56 109.22) (end 165.1 109.22) (width 0.2) (layer "F.Cu") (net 2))
 (segment (start 167.64 116.84) (end 170.18 119.38) (width 0.2) (layer "F.Cu") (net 2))
 (segment (start 170.18 119.38) (end 177.8 119.38) (width 0.2) (layer "F.Cu") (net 2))
 (segment (start 144.74 55.88) (end 144.74 48.3) (width 0.2) (layer "F.Cu") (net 2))
 (segment (start 170.18 142.24) (end 170.18 137.12) (width 0.2) (layer "F.Cu") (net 2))
 (segment (start 165.06 66.04) (end 167.64 66.04) (width 0.2) (layer "F.Cu") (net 2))
 (segment (start 180.3 66.04) (end 180.34 66.04) (width 0.2) (layer "F.Cu") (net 2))
 (segment (start 137.21 116.9) (end 134.56 116.9) (width 0.2) (layer "F.Cu") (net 2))
 (segment (start 180.34 93.98) (end 175.26 93.98) (width 0.2) (layer "F.Cu") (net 2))
 (segment (start 137.16 76.2) (end 137.16 86.36) (width 0.2) (layer "F.Cu") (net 22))
 (segment (start 139.7 73.66) (end 137.16 76.2) (width 0.2) (layer "F.Cu") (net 22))
 (segment (start 132.08 91.44) (end 129.54 91.44) (width 0.2) (layer "F.Cu") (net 22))
 (segment (start 137.16 86.36) (end 132.08 91.44) (width 0.2) (layer "F.Cu") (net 22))
 (segment (start 170.1 124.46) (end 180.34 134.7) (width 0.2) (layer "F.Cu") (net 18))
 (segment (start 170.1 121.92) (end 170.1 124.46) (width 0.2) (layer "F.Cu") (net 18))
 (segment (start 170.1 121.92) (end 144.78 121.92) (width 0.2) (layer "F.Cu") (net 18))
 (segment (start 160.06 73.62) (end 160.02 73.66) (width 0.2) (layer "F.Cu") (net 10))
 (segment (start 160.06 66.04) (end 160.06 73.62) (width 0.2) (layer "F.Cu") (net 10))
 (segment (start 147.32 96.52) (end 144.78 96.52) (width 0.2) (layer "F.Cu") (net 10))
 (segment (start 152.4 78.74) (end 152.4 91.44) (width 0.2) (layer "F.Cu") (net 10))
 (segment (start 157.48 73.66) (end 152.4 78.74) (width 0.2) (layer "F.Cu") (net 10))
 (segment (start 152.4 91.44) (end 147.32 96.52) (width 0.2) (layer "F.Cu") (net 10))
 (segment (start 160.02 73.66) (end 157.48 73.66) (width 0.2) (layer "F.Cu") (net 10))
 (segment (start 160.06 58.38) (end 154.94 63.5) (width 0.2) (layer "F.Cu") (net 9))
 (segment (start 152 63.9) (end 152 89.3) (width 0.2) (layer "F.Cu") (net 9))
 (segment (start 152.4 63.5) (end 152 63.9) (width 0.2) (layer "F.Cu") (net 9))
 (segment (start 154.94 63.5) (end 152.4 63.5) (width 0.2) (layer "F.Cu") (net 9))
 (segment (start 147.32 93.98) (end 144.78 93.98) (width 0.2) (layer "F.Cu") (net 9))
 (segment (start 160.06 53.34) (end 160.06 58.38) (width 0.2) (layer "F.Cu") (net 9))
 (segment (start 152 89.3) (end 147.32 93.98) (width 0.2) (layer "F.Cu") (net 9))
 (segment (start 154.98 116.84) (end 152.44 119.38) (width 0.2) (layer "F.Cu") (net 17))
 (segment (start 152.44 119.38) (end 144.78 119.38) (width 0.2) (layer "F.Cu") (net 17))
 (segment (start 149.86 132.08) (end 149.86 129.54) (width 0.2) (layer "F.Cu") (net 23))
 (segment (start 149.86 129.54) (end 147.32 129.54) (width 0.2) (layer "F.Cu") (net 23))
 (segment (start 132.08 129.54) (end 132.08 121.92) (width 0.2) (layer "F.Cu") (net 23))
 (segment (start 147.32 129.54) (end 132.08 129.54) (width 0.2) (layer "F.Cu") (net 23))
 (segment (start 149.86 134.62) (end 149.86 132.08) (width 0.2) (layer "F.Cu") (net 23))
 (segment (start 154.98 134.62) (end 149.86 134.62) (width 0.2) (layer "F.Cu") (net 23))
 (segment (start 132.08 121.92) (end 130.69 121.92) (width 0.2) (layer "F.Cu") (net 23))
 (segment (start 134.62 123.257919) (end 130.742081 119.38) (width 0.2) (layer "F.Cu") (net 26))
 (segment (start 130.742081 119.38) (end 129.54 119.38) (width 0.2) (layer "F.Cu") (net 26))
 (segment (start 170.18 129.54) (end 167.64 127) (width 0.2) (layer "F.Cu") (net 26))
 (segment (start 134.62 127) (end 134.62 123.257919) (width 0.2) (layer "F.Cu") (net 26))
 (segment (start 167.64 127) (end 134.62 127) (width 0.2) (layer "F.Cu") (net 26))
 (segment (start 170.18 132.12) (end 170.18 129.54) (width 0.2) (layer "F.Cu") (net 26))
 (segment (start 154.94 91.44) (end 154.94 78.74) (width 0.2) (layer "F.Cu") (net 11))
 (segment (start 154.94 78.74) (end 156.795 78.74) (width 0.2) (layer "F.Cu") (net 11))
 (segment (start 147.32 99.06) (end 154.94 91.44) (width 0.2) (layer "F.Cu") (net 11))
 (segment (start 144.78 99.06) (end 147.32 99.06) (width 0.2) (layer "F.Cu") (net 11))
 (segment (start 172.72 78.74) (end 172.72 91.44) (width 0.2) (layer "F.Cu") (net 13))
 (segment (start 152.4 106.68) (end 144.78 106.68) (width 0.2) (layer "F.Cu") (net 13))
 (segment (start 172.72 91.44) (end 160.02 91.44) (width 0.2) (layer "F.Cu") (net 13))
 (segment (start 152.4 99.06) (end 152.4 106.68) (width 0.2) (layer "F.Cu") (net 13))
 (segment (start 160.02 91.44) (end 152.4 99.06) (width 0.2) (layer "F.Cu") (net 13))
 (segment (start 172.8 78.74) (end 172.72 78.74) (width 0.2) (layer "F.Cu") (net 13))
 (segment (start 170.18 71.16) (end 170.18 88.9) (width 0.2) (layer "F.Cu") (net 12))
 (segment (start 149.86 104.14) (end 144.78 104.14) (width 0.2) (layer "F.Cu") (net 12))
 (segment (start 161.994315 88.9) (end 149.86 101.034315) (width 0.2) (layer "F.Cu") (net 12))
 (segment (start 170.18 88.9) (end 161.994315 88.9) (width 0.2) (layer "F.Cu") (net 12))
 (segment (start 175.3 66.04) (end 170.18 71.16) (width 0.2) (layer "F.Cu") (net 12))
 (segment (start 149.86 101.034315) (end 149.86 104.14) (width 0.2) (layer "F.Cu") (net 12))
 (segment (start 147.36 101.6) (end 144.78 101.6) (width 0.2) (layer "F.Cu") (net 3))
 (segment (start 149.9 99.06) (end 147.36 101.6) (width 0.2) (layer "F.Cu") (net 3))
 (segment (start 132.08 93.98) (end 129.54 93.98) (width 0.2) (layer "F.Cu") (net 21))
 (segment (start 137.56 78.34) (end 137.56 88.5) (width 0.2) (layer "F.Cu") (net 21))
 (segment (start 137.56 88.5) (end 132.08 93.98) (width 0.2) (layer "F.Cu") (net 21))
 (segment (start 142.24 73.66) (end 137.56 78.34) (width 0.2) (layer "F.Cu") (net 21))
 (segment (start 135.59316 57.48684) (end 138.13316 57.48684) (width 0.2) (layer "F.Cu") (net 27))
 (segment (start 132.08 70.554314) (end 132.08 81.28) (width 0.2) (layer "F.Cu") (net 27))
 (segment (start 135.59316 57.48684) (end 135.59316 67.041154) (width 0.2) (layer "F.Cu") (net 27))
 (segment (start 132.08 81.28) (end 129.54 81.28) (width 0.2) (layer "F.Cu") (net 27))
 (segment (start 135.59316 67.041154) (end 132.08 70.554314) (width 0.2) (layer "F.Cu") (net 27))
 (segment (start 138.13316 57.48684) (end 139.74 55.88) (width 0.2) (layer "F.Cu") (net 27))
 (segment (start 139.7 78.74) (end 139.7 96.52) (width 0.2) (layer "F.Cu") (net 20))
 (segment (start 144.78 73.66) (end 139.7 78.74) (width 0.2) (layer "F.Cu") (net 20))
 (segment (start 139.7 96.52) (end 129.54 96.52) (width 0.2) (layer "F.Cu") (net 20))
 (segment (start 134.62 114.3) (end 134.62 111.76) (width 0.2) (layer "F.Cu") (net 25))
 (segment (start 132.08 109.22) (end 132.08 101.6) (width 0.2) (layer "F.Cu") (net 25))
 (segment (start 134.62 111.76) (end 132.08 109.22) (width 0.2) (layer "F.Cu") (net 25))
 (segment (start 134.68 114.36) (end 134.62 114.3) (width 0.2) (layer "F.Cu") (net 25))
 (segment (start 132.08 101.6) (end 129.54 101.6) (width 0.2) (layer "F.Cu") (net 25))
 (segment (start 137.21 114.36) (end 134.68 114.36) (width 0.2) (layer "F.Cu") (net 25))
 (segment (start 132.48 99.46) (end 132.08 99.06) (width 0.2) (layer "F.Cu") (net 24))
 (segment (start 137.21 109.28) (end 132.705686 109.28) (width 0.2) (layer "F.Cu") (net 24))
 (segment (start 132.705686 109.28) (end 132.48 109.054314) (width 0.2) (layer "F.Cu") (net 24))
 (segment (start 132.08 99.06) (end 129.54 99.06) (width 0.2) (layer "F.Cu") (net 24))
 (segment (start 132.48 109.054314) (end 132.48 99.46) (width 0.2) (layer "F.Cu") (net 24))
 (segment (start 167.68 99.06) (end 165.5 99.06) (width 0.2) (layer "F.Cu") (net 15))
 (segment (start 165.5 99.06) (end 165.5 113.9) (width 0.2) (layer "F.Cu") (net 15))
 (segment (start 165.1 114.3) (end 144.78 114.3) (width 0.2) (layer "F.Cu") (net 15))
 (segment (start 165.5 113.9) (end 165.1 114.3) (width 0.2) (layer "F.Cu") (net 15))
 (segment (start 171.706 115.786) (end 145.834 115.786) (width 0.2) (layer "F.Cu") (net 16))
 (segment (start 172.76 116.84) (end 171.706 115.786) (width 0.2) (layer "F.Cu") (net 16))
 (segment (start 145.834 115.786) (end 144.78 116.84) (width 0.2) (layer "F.Cu") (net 16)))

